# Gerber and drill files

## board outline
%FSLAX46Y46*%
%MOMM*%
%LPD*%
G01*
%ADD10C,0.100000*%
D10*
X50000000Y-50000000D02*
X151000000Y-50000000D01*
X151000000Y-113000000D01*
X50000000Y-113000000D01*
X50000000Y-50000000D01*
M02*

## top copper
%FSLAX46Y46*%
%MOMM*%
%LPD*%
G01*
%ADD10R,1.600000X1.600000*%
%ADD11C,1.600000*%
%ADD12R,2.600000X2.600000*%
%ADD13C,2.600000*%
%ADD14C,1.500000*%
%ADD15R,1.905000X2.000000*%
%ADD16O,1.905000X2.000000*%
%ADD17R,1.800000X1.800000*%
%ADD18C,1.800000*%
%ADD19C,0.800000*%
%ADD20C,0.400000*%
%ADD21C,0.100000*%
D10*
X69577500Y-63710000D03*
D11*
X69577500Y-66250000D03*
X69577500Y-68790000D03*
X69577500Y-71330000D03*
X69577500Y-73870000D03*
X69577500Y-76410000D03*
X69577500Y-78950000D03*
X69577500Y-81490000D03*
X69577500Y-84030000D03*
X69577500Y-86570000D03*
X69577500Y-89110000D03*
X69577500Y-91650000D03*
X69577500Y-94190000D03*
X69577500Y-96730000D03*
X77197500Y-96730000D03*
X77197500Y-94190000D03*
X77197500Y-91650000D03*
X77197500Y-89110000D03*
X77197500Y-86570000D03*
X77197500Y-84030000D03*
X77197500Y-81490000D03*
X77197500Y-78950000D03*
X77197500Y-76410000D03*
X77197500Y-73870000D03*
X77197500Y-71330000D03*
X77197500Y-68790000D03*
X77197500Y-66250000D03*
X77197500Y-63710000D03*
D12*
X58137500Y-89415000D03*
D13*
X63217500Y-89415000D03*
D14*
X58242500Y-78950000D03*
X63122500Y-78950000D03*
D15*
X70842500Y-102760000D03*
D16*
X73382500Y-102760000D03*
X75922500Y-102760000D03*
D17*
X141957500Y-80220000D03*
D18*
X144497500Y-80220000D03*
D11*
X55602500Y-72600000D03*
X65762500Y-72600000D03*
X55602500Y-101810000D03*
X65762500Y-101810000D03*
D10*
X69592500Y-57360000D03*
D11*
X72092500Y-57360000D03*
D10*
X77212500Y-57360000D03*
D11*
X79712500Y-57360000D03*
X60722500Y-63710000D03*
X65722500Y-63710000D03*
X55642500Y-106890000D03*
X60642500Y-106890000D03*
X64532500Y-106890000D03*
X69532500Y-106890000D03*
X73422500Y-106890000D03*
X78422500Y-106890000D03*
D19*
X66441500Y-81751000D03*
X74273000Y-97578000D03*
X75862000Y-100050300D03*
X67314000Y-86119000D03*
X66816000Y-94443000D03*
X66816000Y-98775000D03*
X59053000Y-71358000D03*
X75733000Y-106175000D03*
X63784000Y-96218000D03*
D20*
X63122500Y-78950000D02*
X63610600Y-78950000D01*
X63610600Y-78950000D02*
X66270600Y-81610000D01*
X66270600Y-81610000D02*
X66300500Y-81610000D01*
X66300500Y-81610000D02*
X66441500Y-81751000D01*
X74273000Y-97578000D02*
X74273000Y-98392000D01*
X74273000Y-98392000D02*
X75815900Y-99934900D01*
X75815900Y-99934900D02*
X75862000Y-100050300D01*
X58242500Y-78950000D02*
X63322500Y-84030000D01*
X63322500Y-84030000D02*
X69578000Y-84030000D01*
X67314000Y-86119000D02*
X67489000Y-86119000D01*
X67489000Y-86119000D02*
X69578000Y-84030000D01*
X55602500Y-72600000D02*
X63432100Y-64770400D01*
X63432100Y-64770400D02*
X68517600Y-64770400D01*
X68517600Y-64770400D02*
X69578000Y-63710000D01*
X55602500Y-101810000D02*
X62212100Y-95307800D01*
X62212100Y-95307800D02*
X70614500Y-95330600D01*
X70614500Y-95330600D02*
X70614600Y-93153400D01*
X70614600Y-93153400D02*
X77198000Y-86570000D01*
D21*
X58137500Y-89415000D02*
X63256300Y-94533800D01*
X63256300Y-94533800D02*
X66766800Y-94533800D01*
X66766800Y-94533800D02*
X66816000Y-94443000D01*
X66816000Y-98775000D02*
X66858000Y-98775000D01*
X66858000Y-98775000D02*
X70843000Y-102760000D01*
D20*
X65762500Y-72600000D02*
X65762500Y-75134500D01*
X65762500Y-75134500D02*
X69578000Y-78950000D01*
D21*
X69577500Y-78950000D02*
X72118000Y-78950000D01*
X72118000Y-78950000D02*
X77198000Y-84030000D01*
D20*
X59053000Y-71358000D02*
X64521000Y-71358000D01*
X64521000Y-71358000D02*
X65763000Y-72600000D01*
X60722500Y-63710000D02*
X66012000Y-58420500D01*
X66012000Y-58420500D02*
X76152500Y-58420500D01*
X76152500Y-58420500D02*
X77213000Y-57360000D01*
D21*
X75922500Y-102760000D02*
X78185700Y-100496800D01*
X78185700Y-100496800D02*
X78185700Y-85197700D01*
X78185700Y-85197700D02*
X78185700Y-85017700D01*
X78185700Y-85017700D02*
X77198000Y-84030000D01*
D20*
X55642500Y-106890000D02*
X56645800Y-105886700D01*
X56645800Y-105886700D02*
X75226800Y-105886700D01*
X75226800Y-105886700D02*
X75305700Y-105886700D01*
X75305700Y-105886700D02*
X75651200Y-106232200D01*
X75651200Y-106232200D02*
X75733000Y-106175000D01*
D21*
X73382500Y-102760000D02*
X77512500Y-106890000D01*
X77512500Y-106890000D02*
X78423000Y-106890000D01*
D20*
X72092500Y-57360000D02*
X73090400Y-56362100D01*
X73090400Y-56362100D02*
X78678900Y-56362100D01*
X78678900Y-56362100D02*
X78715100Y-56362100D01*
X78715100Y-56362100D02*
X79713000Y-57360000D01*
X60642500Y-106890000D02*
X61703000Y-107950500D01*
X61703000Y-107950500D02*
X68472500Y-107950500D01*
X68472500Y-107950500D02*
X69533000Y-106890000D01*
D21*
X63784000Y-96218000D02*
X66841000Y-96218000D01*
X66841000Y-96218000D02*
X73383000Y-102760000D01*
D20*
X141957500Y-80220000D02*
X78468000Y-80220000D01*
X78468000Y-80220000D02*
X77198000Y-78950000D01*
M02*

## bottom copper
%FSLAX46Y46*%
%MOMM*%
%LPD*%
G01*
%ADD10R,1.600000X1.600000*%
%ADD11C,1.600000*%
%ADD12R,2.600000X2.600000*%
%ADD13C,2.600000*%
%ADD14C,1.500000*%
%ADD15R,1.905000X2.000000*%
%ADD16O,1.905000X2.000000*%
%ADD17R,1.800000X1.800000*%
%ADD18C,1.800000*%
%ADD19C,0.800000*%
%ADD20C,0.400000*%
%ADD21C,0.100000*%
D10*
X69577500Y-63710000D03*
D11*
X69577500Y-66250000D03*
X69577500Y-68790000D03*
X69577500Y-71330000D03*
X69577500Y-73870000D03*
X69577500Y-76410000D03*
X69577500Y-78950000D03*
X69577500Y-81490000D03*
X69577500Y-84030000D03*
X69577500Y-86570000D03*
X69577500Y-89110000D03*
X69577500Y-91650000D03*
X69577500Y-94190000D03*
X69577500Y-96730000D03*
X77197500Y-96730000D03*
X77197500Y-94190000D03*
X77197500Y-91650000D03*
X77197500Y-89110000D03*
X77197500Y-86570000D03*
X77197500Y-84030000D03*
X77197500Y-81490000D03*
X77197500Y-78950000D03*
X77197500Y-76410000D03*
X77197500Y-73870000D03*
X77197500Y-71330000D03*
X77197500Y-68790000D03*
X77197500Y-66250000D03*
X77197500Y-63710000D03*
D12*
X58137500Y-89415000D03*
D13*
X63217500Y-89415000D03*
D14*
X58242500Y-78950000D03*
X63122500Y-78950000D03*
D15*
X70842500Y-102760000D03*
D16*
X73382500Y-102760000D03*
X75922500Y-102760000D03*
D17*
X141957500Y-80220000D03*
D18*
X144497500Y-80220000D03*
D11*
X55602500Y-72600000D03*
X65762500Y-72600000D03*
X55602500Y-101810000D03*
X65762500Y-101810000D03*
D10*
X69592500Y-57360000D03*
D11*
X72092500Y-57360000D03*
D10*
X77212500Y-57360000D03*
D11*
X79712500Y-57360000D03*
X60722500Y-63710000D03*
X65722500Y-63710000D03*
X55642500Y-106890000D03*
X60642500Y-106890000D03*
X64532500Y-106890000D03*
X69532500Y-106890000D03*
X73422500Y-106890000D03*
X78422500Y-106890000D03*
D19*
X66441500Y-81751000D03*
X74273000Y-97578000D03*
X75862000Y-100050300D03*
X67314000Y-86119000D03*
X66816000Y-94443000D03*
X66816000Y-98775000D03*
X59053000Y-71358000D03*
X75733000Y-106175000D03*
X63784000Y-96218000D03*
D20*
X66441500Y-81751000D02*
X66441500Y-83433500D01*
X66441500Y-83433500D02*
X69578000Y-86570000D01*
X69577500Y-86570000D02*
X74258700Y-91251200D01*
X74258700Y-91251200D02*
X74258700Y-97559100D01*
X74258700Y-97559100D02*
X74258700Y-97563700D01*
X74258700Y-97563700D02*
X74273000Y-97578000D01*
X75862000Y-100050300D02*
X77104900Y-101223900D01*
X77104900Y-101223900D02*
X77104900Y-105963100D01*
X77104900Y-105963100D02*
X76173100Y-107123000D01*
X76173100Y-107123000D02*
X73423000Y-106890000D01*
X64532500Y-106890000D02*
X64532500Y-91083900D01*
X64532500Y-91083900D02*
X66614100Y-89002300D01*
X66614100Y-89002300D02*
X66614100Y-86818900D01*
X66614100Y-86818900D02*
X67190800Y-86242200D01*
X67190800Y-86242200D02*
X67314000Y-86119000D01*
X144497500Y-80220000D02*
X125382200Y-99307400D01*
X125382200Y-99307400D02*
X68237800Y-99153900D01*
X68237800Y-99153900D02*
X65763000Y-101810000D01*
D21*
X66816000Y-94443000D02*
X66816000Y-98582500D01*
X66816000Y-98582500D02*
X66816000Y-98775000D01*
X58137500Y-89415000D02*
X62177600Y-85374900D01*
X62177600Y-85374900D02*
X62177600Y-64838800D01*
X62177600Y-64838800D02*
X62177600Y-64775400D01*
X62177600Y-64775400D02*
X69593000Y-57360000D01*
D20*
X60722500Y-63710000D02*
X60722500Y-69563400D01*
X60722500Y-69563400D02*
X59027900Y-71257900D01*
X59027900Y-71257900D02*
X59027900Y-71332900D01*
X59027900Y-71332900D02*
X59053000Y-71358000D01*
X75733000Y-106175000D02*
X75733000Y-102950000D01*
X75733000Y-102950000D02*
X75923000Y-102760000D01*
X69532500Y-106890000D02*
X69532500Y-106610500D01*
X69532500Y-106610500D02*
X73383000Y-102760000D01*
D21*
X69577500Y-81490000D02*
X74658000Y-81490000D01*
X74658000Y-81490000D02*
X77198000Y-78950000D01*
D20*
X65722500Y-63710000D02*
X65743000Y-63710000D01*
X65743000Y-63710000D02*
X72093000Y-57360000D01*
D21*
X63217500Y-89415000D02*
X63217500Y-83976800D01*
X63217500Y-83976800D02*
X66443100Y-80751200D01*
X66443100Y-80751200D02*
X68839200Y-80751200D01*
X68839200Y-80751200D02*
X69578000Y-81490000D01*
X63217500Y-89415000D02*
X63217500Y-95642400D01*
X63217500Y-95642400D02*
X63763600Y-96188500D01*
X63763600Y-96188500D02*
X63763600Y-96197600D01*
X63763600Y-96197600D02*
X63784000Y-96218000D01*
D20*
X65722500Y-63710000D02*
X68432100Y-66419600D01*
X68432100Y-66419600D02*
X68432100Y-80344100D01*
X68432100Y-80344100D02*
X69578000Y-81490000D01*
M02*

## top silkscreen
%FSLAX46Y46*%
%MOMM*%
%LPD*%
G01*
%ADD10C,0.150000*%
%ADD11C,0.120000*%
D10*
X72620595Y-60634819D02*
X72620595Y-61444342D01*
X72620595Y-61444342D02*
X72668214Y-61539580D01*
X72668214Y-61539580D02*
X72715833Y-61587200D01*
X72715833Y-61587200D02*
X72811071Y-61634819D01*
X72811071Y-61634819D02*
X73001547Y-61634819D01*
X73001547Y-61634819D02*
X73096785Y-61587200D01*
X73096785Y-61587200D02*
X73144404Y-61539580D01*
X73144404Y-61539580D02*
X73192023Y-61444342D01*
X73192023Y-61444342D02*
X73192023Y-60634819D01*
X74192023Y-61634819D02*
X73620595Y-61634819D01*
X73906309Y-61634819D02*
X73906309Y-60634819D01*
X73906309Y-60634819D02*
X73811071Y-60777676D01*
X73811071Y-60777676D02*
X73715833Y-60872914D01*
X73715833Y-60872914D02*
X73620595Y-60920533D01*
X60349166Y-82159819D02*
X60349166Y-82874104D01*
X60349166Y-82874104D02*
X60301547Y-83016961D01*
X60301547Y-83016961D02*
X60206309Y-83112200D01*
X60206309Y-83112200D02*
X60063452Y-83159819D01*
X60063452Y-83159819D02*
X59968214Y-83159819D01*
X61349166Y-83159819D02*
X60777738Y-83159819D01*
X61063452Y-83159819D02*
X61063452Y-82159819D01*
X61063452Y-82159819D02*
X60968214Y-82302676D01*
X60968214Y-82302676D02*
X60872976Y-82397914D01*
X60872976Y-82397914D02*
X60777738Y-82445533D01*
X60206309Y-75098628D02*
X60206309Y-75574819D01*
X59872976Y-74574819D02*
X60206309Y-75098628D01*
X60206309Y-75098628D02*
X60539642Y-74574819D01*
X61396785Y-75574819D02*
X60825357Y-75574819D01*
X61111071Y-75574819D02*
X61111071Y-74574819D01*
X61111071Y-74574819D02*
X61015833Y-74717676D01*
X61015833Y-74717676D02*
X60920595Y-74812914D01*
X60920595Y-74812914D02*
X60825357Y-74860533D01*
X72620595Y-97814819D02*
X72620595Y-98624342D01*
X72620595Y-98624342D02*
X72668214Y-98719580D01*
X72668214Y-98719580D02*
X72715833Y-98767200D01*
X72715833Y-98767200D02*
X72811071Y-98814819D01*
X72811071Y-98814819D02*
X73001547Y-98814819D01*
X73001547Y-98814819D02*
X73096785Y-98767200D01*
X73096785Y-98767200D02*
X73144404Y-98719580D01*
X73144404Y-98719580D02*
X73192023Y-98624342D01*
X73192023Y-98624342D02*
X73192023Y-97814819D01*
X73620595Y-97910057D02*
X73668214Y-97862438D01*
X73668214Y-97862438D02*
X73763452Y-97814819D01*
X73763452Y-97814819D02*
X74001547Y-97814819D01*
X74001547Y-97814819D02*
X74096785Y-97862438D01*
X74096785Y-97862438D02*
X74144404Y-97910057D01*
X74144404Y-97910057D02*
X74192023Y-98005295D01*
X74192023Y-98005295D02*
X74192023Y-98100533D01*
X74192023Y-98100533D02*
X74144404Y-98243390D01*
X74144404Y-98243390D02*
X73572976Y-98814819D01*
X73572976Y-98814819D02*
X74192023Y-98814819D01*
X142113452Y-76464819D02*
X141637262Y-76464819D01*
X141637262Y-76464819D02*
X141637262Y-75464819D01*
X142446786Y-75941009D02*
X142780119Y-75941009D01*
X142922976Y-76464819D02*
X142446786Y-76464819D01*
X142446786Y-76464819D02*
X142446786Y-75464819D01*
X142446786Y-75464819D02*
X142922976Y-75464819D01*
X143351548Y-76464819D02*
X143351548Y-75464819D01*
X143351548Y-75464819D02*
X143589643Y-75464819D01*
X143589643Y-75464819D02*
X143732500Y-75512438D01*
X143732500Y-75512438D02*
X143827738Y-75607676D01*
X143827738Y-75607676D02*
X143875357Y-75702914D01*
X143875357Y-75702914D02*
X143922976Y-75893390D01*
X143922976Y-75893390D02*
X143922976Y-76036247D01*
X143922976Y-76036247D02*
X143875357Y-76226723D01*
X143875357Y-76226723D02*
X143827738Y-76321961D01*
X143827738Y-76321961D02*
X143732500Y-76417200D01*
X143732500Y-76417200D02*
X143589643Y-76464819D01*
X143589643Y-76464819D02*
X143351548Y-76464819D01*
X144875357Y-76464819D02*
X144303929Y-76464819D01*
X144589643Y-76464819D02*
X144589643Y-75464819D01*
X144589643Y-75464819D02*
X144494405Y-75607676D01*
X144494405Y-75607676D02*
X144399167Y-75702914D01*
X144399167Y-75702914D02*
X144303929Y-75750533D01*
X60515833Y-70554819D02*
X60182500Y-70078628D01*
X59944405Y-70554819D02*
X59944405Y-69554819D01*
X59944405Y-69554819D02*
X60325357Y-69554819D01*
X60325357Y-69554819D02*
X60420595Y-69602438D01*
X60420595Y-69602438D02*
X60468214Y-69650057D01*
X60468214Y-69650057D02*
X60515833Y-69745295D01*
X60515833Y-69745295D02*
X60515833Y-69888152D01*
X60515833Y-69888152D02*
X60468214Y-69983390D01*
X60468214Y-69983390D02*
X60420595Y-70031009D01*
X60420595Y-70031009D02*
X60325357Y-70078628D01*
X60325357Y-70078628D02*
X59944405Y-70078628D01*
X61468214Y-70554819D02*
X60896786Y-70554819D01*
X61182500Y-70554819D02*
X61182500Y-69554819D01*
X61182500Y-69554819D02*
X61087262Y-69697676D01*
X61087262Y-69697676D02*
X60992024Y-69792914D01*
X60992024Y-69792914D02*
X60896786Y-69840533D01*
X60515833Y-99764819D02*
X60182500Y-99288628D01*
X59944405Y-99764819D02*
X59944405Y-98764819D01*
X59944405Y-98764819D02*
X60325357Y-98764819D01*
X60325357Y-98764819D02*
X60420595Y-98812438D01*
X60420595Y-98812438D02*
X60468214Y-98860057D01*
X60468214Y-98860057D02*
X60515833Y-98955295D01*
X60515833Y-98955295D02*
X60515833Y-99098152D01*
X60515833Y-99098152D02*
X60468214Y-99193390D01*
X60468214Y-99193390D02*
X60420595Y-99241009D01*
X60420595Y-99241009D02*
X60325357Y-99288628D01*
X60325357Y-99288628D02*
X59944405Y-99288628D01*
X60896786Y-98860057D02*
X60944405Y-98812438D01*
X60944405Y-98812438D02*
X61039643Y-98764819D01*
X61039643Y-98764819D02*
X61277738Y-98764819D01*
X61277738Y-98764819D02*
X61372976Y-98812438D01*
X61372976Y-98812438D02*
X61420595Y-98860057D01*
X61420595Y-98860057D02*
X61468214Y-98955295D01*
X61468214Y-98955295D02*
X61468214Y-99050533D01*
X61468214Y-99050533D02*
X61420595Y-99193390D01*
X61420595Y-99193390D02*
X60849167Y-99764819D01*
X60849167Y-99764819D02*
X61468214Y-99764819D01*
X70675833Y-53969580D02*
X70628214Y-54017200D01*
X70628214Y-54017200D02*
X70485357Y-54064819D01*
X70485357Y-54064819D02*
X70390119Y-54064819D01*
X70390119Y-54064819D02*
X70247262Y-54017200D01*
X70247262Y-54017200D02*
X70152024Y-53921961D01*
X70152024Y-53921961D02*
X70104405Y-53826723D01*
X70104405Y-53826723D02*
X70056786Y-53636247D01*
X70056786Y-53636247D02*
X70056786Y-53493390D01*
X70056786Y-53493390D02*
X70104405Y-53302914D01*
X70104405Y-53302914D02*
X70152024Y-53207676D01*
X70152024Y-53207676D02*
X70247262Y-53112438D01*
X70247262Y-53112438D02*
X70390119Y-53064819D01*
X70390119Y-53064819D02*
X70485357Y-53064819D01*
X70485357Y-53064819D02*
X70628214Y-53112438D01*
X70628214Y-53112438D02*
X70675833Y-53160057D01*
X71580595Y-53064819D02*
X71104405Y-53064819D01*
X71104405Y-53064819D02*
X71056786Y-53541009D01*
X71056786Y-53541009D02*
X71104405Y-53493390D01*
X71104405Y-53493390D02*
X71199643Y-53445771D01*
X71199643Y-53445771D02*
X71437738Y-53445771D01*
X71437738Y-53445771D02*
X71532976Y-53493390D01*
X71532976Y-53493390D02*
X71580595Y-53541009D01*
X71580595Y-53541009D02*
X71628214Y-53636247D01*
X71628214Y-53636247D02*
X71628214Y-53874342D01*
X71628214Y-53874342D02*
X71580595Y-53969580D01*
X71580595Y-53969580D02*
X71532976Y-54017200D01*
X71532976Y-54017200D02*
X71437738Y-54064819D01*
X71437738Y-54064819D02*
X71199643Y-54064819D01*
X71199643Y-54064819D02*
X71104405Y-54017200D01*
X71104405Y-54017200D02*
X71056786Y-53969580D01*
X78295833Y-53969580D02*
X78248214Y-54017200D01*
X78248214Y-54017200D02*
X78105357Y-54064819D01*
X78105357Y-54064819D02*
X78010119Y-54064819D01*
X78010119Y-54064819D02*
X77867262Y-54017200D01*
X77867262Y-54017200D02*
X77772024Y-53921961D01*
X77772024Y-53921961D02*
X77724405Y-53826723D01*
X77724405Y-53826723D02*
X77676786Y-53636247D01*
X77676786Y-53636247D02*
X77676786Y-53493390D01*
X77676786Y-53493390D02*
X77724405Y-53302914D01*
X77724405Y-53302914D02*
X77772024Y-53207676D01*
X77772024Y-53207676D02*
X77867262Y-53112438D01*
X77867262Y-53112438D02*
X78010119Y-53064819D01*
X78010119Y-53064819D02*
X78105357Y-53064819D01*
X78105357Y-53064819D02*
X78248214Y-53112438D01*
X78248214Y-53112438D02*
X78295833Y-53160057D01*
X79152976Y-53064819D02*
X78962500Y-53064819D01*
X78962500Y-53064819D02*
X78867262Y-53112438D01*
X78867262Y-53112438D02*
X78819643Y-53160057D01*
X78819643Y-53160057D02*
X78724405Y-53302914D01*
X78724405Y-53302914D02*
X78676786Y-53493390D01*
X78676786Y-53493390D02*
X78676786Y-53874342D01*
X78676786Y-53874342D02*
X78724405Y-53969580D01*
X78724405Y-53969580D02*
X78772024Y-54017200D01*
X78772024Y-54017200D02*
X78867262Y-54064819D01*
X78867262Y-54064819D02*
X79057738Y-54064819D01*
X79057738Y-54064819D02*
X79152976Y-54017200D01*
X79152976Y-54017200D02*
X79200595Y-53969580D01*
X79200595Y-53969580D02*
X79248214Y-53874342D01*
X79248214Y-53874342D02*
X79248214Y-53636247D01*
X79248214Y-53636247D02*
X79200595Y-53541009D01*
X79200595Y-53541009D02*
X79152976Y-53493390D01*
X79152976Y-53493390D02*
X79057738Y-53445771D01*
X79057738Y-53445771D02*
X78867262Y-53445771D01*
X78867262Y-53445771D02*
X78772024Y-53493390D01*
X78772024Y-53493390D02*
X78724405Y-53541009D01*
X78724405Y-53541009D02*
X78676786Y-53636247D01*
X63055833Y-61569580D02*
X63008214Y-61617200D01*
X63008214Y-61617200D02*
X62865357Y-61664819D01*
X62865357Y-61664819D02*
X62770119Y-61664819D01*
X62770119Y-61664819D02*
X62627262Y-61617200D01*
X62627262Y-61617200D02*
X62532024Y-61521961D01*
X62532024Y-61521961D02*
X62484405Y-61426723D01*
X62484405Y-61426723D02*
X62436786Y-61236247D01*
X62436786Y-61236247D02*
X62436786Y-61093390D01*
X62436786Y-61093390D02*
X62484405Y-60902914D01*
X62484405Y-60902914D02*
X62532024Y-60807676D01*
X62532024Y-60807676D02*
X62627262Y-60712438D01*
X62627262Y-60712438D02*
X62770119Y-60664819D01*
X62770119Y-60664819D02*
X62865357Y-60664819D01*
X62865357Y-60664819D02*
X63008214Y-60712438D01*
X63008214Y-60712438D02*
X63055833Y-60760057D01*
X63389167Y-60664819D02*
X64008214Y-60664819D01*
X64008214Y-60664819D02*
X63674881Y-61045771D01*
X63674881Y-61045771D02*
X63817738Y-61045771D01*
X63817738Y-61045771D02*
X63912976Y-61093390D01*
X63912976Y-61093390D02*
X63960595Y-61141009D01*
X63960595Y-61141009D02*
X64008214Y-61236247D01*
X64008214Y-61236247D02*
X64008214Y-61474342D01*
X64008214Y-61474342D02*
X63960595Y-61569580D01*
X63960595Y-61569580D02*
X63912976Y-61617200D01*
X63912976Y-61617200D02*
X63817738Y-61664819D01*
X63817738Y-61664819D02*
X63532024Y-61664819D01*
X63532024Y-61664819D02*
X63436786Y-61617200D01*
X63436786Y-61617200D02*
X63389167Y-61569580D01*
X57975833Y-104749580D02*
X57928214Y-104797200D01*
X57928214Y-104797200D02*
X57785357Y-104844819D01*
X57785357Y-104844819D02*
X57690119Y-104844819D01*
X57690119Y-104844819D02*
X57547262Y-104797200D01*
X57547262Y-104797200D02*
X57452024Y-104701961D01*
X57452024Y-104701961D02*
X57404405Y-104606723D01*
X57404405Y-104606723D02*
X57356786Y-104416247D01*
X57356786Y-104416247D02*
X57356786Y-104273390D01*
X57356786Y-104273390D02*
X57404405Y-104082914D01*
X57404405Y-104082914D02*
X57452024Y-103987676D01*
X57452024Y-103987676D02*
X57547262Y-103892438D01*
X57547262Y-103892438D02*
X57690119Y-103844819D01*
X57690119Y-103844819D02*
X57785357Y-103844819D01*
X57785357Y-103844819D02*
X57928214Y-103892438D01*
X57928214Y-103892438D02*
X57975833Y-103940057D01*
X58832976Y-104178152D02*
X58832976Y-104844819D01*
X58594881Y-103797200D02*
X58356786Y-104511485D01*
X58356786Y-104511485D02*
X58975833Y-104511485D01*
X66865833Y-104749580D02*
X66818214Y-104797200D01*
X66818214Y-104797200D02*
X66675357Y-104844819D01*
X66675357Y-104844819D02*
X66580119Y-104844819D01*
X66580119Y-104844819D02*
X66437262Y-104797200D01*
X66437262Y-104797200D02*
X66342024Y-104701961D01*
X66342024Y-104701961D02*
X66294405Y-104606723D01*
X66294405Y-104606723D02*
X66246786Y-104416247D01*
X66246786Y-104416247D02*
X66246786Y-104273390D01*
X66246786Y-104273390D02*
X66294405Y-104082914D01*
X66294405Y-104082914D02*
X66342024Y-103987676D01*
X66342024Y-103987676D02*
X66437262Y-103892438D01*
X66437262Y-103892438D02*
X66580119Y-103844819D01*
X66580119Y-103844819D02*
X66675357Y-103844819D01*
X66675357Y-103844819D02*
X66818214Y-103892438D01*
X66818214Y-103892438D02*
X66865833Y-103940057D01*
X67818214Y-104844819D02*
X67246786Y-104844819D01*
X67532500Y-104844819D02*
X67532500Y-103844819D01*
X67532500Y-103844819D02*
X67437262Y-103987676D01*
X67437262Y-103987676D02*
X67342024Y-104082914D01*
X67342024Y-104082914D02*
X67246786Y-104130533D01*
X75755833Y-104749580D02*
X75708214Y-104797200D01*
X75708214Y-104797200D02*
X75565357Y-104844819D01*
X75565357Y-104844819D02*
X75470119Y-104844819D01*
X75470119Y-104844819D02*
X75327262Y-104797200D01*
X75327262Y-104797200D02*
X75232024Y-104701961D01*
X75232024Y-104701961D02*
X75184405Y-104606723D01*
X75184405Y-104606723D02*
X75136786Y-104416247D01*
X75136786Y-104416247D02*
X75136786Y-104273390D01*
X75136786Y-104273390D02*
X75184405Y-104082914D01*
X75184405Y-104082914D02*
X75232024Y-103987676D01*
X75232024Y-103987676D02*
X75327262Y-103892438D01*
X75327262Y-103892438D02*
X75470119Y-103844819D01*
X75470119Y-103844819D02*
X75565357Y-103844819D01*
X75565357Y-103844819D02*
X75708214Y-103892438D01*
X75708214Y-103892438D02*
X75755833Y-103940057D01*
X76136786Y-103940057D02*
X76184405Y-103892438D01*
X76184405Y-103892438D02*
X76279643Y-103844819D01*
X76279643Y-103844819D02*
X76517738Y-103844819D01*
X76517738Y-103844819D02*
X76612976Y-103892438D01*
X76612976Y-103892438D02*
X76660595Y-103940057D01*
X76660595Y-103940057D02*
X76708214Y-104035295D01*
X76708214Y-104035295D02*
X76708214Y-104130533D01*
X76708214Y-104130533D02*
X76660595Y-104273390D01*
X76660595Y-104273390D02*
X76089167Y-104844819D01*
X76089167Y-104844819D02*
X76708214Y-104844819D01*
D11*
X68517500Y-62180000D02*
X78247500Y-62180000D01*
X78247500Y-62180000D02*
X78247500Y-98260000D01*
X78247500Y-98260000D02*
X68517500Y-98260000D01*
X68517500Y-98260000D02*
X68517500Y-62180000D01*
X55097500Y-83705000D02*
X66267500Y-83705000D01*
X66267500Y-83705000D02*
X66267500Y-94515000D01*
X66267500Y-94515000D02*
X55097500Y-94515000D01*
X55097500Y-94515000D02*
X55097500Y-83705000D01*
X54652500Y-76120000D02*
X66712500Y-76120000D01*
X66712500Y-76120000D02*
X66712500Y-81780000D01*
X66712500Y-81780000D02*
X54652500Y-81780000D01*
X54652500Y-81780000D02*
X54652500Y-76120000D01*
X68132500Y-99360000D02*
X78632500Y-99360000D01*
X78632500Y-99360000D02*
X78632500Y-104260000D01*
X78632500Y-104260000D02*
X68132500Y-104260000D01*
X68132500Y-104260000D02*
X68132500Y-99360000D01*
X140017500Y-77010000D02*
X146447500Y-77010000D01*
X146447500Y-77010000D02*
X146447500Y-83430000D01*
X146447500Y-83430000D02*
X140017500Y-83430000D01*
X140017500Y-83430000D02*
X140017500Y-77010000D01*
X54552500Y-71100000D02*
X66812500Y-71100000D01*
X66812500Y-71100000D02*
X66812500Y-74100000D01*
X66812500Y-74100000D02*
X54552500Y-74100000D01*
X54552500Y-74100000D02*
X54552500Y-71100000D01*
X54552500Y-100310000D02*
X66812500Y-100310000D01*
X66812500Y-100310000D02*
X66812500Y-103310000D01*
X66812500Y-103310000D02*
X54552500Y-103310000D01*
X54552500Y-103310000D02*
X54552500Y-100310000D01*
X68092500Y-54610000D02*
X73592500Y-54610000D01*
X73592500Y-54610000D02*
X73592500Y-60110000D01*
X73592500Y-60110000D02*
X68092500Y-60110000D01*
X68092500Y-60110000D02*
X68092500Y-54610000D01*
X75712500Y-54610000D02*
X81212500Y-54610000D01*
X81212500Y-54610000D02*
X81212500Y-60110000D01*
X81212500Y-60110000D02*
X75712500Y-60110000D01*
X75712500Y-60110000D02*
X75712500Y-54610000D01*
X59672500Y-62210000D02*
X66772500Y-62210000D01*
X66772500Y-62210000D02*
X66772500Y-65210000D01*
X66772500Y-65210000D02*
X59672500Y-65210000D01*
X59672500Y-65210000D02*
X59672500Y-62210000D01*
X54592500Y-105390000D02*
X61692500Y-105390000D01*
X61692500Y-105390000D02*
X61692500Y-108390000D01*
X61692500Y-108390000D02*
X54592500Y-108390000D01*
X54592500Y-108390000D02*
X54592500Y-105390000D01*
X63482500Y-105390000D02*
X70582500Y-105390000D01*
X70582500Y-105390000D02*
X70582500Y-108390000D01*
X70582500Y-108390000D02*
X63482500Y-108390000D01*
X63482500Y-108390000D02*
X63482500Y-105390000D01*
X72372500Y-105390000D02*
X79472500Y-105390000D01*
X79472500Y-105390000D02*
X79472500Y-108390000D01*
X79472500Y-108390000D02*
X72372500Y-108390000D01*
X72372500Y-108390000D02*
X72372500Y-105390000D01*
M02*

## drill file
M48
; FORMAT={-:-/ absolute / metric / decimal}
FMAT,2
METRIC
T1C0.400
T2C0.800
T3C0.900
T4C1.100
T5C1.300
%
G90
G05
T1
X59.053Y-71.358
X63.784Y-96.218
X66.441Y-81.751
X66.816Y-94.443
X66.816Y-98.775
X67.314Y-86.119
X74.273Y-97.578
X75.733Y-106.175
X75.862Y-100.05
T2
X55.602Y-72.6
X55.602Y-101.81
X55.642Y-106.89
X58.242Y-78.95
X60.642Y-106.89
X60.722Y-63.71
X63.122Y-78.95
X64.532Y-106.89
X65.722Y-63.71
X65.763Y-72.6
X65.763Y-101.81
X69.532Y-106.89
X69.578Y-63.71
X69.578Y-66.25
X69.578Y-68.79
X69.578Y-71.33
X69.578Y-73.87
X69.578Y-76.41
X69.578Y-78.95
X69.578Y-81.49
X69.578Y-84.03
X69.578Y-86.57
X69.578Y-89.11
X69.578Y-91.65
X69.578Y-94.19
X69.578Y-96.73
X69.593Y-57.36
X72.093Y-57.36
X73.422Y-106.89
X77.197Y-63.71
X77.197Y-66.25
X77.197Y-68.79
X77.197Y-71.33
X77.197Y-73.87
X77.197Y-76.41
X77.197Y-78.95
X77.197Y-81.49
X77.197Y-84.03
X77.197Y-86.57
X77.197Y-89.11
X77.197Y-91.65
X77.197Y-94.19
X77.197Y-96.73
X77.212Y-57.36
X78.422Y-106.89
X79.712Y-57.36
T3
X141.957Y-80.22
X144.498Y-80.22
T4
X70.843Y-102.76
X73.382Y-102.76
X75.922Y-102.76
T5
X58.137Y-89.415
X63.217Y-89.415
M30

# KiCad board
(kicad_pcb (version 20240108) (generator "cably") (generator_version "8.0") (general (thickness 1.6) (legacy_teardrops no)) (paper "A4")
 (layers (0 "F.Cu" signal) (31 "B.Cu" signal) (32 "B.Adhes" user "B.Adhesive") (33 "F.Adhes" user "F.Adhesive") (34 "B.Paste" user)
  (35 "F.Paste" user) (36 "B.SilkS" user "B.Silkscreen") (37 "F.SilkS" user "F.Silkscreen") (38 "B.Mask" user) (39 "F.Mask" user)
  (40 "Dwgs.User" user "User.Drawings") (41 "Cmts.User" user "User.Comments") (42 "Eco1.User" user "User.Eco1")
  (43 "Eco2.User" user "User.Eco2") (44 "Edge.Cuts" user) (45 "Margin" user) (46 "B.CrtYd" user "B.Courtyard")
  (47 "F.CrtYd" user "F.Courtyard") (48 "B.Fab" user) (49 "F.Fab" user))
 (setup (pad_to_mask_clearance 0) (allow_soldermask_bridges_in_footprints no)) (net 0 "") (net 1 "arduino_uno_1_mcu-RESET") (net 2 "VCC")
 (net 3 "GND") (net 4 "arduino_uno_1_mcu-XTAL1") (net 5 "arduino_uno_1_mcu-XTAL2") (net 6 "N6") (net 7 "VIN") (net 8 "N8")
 (gr_rect (start 50 50) (end 151 113) (stroke (width 0.1) (type default)) (fill none) (layer "Edge.Cuts"))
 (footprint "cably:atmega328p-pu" (layer "F.Cu") (at 73.3825 80.22)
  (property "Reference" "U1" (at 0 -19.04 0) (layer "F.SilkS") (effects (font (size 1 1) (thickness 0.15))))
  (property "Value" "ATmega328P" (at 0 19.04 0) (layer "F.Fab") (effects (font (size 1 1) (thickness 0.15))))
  (fp_line (start -4.865 -18.04) (end 4.865 -18.04) (stroke (width 0.12) (type solid)) (layer "F.SilkS"))
  (fp_line (start 4.865 -18.04) (end 4.865 18.04) (stroke (width 0.12) (type solid)) (layer "F.SilkS"))
  (fp_line (start 4.865 18.04) (end -4.865 18.04) (stroke (width 0.12) (type solid)) (layer "F.SilkS"))
  (fp_line (start -4.865 18.04) (end -4.865 -18.04) (stroke (width 0.12) (type solid)) (layer "F.SilkS"))
  (pad "1" thru_hole rect (at -3.805 -16.51) (size 1.6 1.6) (drill 0.8) (layers "*.Cu" "*.Mask") (remove_unused_layers no)
   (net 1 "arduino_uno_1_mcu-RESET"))
  (pad "2" thru_hole circle (at -3.805 -13.97) (size 1.6 1.6) (drill 0.8) (layers "*.Cu" "*.Mask") (remove_unused_layers no))
  (pad "3" thru_hole circle (at -3.805 -11.43) (size 1.6 1.6) (drill 0.8) (layers "*.Cu" "*.Mask") (remove_unused_layers no))
  (pad "4" thru_hole circle (at -3.805 -8.89) (size 1.6 1.6) (drill 0.8) (layers "*.Cu" "*.Mask") (remove_unused_layers no))
  (pad "5" thru_hole circle (at -3.805 -6.35) (size 1.6 1.6) (drill 0.8) (layers "*.Cu" "*.Mask") (remove_unused_layers no))
  (pad "6" thru_hole circle (at -3.805 -3.81) (size 1.6 1.6) (drill 0.8) (layers "*.Cu" "*.Mask") (remove_unused_layers no))
  (pad "7" thru_hole circle (at -3.805 -1.27) (size 1.6 1.6) (drill 0.8) (layers "*.Cu" "*.Mask") (remove_unused_layers no) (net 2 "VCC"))
  (pad "8" thru_hole circle (at -3.805 1.27) (size 1.6 1.6) (drill 0.8) (layers "*.Cu" "*.Mask") (remove_unused_layers no) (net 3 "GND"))
  (pad "9" thru_hole circle (at -3.805 3.81) (size 1.6 1.6) (drill 0.8) (layers "*.Cu" "*.Mask") (remove_unused_layers no)
   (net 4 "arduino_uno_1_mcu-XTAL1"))
  (pad "10" thru_hole circle (at -3.805 6.35) (size 1.6 1.6) (drill 0.8) (layers "*.Cu" "*.Mask") (remove_unused_layers no)
   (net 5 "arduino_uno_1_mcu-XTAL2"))
  (pad "11" thru_hole circle (at -3.805 8.89) (size 1.6 1.6) (drill 0.8) (layers "*.Cu" "*.Mask") (remove_unused_layers no))
  (pad "12" thru_hole circle (at -3.805 11.43) (size 1.6 1.6) (drill 0.8) (layers "*.Cu" "*.Mask") (remove_unused_layers no))
  (pad "13" thru_hole circle (at -3.805 13.97) (size 1.6 1.6) (drill 0.8) (layers "*.Cu" "*.Mask") (remove_unused_layers no))
  (pad "14" thru_hole circle (at -3.805 16.51) (size 1.6 1.6) (drill 0.8) (layers "*.Cu" "*.Mask") (remove_unused_layers no))
  (pad "15" thru_hole circle (at 3.815 16.51) (size 1.6 1.6) (drill 0.8) (layers "*.Cu" "*.Mask") (remove_unused_layers no))
  (pad "16" thru_hole circle (at 3.815 13.97) (size 1.6 1.6) (drill 0.8) (layers "*.Cu" "*.Mask") (remove_unused_layers no))
  (pad "17" thru_hole circle (at 3.815 11.43) (size 1.6 1.6) (drill 0.8) (layers "*.Cu" "*.Mask") (remove_unused_layers no))
  (pad "18" thru_hole circle (at 3.815 8.89) (size 1.6 1.6) (drill 0.8) (layers "*.Cu" "*.Mask") (remove_unused_layers no))
  (pad "19" thru_hole circle (at 3.815 6.35) (size 1.6 1.6) (drill 0.8) (layers "*.Cu" "*.Mask") (remove_unused_layers no) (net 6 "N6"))
  (pad "20" thru_hole circle (at 3.815 3.81) (size 1.6 1.6) (drill 0.8) (layers "*.Cu" "*.Mask") (remove_unused_layers no) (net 2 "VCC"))
  (pad "21" thru_hole circle (at 3.815 1.27) (size 1.6 1.6) (drill 0.8) (layers "*.Cu" "*.Mask") (remove_unused_layers no))
  (pad "22" thru_hole circle (at 3.815 -1.27) (size 1.6 1.6) (drill 0.8) (layers "*.Cu" "*.Mask") (remove_unused_layers no) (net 3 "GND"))
  (pad "23" thru_hole circle (at 3.815 -3.81) (size 1.6 1.6) (drill 0.8) (layers "*.Cu" "*.Mask") (remove_unused_layers no))
  (pad "24" thru_hole circle (at 3.815 -6.35) (size 1.6 1.6) (drill 0.8) (layers "*.Cu" "*.Mask") (remove_unused_layers no))
  (pad "25" thru_hole circle (at 3.815 -8.89) (size 1.6 1.6) (drill 0.8) (layers "*.Cu" "*.Mask") (remove_unused_layers no))
  (pad "26" thru_hole circle (at 3.815 -11.43) (size 1.6 1.6) (drill 0.8) (layers "*.Cu" "*.Mask") (remove_unused_layers no))
  (pad "27" thru_hole circle (at 3.815 -13.97) (size 1.6 1.6) (drill 0.8) (layers "*.Cu" "*.Mask") (remove_unused_layers no))
  (pad "28" thru_hole circle (at 3.815 -16.51) (size 1.6 1.6) (drill 0.8) (layers "*.Cu" "*.Mask") (remove_unused_layers no)))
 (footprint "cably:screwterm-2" (layer "F.Cu") (at 60.6825 89.11)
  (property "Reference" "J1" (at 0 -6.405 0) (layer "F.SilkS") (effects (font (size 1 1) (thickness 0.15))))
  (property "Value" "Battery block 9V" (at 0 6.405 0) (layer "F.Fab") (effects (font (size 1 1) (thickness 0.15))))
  (fp_line (start -5.585 -5.405) (end 5.585 -5.405) (stroke (width 0.12) (type solid)) (layer "F.SilkS"))
  (fp_line (start 5.585 -5.405) (end 5.585 5.405) (stroke (width 0.12) (type solid)) (layer "F.SilkS"))
  (fp_line (start 5.585 5.405) (end -5.585 5.405) (stroke (width 0.12) (type solid)) (layer "F.SilkS"))
  (fp_line (start -5.585 5.405) (end -5.585 -5.405) (stroke (width 0.12) (type solid)) (layer "F.SilkS"))
  (pad "1" thru_hole rect (at -2.545 0.305) (size 2.6 2.6) (drill 1.3) (layers "*.Cu" "*.Mask") (remove_unused_layers no) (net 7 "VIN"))
  (pad "2" thru_hole circle (at 2.535 0.305) (size 2.6 2.6) (drill 1.3) (layers "*.Cu" "*.Mask") (remove_unused_layers no) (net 3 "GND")))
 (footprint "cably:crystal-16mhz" (layer "F.Cu") (at 60.6825 78.95)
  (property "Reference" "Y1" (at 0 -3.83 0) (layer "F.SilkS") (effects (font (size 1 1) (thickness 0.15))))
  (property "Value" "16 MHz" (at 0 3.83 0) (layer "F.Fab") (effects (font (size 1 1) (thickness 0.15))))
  (fp_line (start -6.03 -2.83) (end 6.03 -2.83) (stroke (width 0.12) (type solid)) (layer "F.SilkS"))
  (fp_line (start 6.03 -2.83) (end 6.03 2.83) (stroke (width 0.12) (type solid)) (layer "F.SilkS"))
  (fp_line (start 6.03 2.83) (end -6.03 2.83) (stroke (width 0.12) (type solid)) (layer "F.SilkS"))
  (fp_line (start -6.03 2.83) (end -6.03 -2.83) (stroke (width 0.12) (type solid)) (layer "F.SilkS"))
  (pad "1" thru_hole circle (at -2.44 0) (size 1.5 1.5) (drill 0.8) (layers "*.Cu" "*.Mask") (remove_unused_layers no)
   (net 4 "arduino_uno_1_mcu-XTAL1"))
  (pad "2" thru_hole circle (at 2.44 0) (size 1.5 1.5) (drill 0.8) (layers "*.Cu" "*.Mask") (remove_unused_layers no)
   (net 5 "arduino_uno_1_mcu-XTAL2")))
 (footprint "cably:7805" (layer "F.Cu") (at 73.3825 101.81)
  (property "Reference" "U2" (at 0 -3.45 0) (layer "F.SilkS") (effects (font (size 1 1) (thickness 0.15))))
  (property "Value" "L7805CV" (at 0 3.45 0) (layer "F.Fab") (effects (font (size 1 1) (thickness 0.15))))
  (fp_line (start -5.25 -2.45) (end 5.25 -2.45) (stroke (width 0.12) (type solid)) (layer "F.SilkS"))
  (fp_line (start 5.25 -2.45) (end 5.25 2.45) (stroke (width 0.12) (type solid)) (layer "F.SilkS"))
  (fp_line (start 5.25 2.45) (end -5.25 2.45) (stroke (width 0.12) (type solid)) (layer "F.SilkS"))
  (fp_line (start -5.25 2.45) (end -5.25 -2.45) (stroke (width 0.12) (type solid)) (layer "F.SilkS"))
  (pad "1" thru_hole rect (at -2.54 0.95) (size 1.905 2) (drill 1.1) (layers "*.Cu" "*.Mask") (remove_unused_layers no) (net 7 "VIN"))
  (pad "2" thru_hole oval (at 0 0.95) (size 1.905 2) (drill 1.1) (layers "*.Cu" "*.Mask") (remove_unused_layers no) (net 3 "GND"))
  (pad "3" thru_hole oval (at 2.54 0.95) (size 1.905 2) (drill 1.1) (layers "*.Cu" "*.Mask") (remove_unused_layers no) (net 2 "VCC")))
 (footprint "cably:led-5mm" (layer "F.Cu") (at 143.2325 80.22)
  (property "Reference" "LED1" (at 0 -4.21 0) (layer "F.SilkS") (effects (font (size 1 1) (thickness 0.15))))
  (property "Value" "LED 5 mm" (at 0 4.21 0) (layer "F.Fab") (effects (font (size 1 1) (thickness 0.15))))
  (fp_line (start -3.215 -3.21) (end 3.215 -3.21) (stroke (width 0.12) (type solid)) (layer "F.SilkS"))
  (fp_line (start 3.215 -3.21) (end 3.215 3.21) (stroke (width 0.12) (type solid)) (layer "F.SilkS"))
  (fp_line (start 3.215 3.21) (end -3.215 3.21) (stroke (width 0.12) (type solid)) (layer "F.SilkS"))
  (fp_line (start -3.215 3.21) (end -3.215 -3.21) (stroke (width 0.12) (type solid)) (layer "F.SilkS"))
  (pad "1" thru_hole rect (at -1.275 0) (size 1.8 1.8) (drill 0.9) (layers "*.Cu" "*.Mask") (remove_unused_layers no) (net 3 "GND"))
  (pad "2" thru_hole circle (at 1.265 0) (size 1.8 1.8) (drill 0.9) (layers "*.Cu" "*.Mask") (remove_unused_layers no) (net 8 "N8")))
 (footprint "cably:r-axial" (layer "F.Cu") (at 60.6825 72.6)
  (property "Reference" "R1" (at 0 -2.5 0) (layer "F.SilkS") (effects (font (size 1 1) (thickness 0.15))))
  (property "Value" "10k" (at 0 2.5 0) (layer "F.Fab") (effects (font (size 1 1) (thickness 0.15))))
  (fp_line (start -6.13 -1.5) (end 6.13 -1.5) (stroke (width 0.12) (type solid)) (layer "F.SilkS"))
  (fp_line (start 6.13 -1.5) (end 6.13 1.5) (stroke (width 0.12) (type solid)) (layer "F.SilkS"))
  (fp_line (start 6.13 1.5) (end -6.13 1.5) (stroke (width 0.12) (type solid)) (layer "F.SilkS"))
  (fp_line (start -6.13 1.5) (end -6.13 -1.5) (stroke (width 0.12) (type solid)) (layer "F.SilkS"))
  (pad "1" thru_hole circle (at -5.08 0) (size 1.6 1.6) (drill 0.8) (layers "*.Cu" "*.Mask") (remove_unused_layers no)
   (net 1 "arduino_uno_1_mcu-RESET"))
  (pad "2" thru_hole circle (at 5.08 0) (size 1.6 1.6) (drill 0.8) (layers "*.Cu" "*.Mask") (remove_unused_layers no) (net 2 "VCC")))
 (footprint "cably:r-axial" (layer "F.Cu") (at 60.6825 101.81)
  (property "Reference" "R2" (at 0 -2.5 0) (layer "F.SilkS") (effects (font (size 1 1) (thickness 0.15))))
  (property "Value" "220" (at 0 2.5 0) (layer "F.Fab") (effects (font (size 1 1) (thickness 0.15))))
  (fp_line (start -6.13 -1.5) (end 6.13 -1.5) (stroke (width 0.12) (type solid)) (layer "F.SilkS"))
  (fp_line (start 6.13 -1.5) (end 6.13 1.5) (stroke (width 0.12) (type solid)) (layer "F.SilkS"))
  (fp_line (start 6.13 1.5) (end -6.13 1.5) (stroke (width 0.12) (type solid)) (layer "F.SilkS"))
  (fp_line (start -6.13 1.5) (end -6.13 -1.5) (stroke (width 0.12) (type solid)) (layer "F.SilkS"))
  (pad "1" thru_hole circle (at -5.08 0) (size 1.6 1.6) (drill 0.8) (layers "*.Cu" "*.Mask") (remove_unused_layers no) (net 6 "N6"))
  (pad "2" thru_hole circle (at 5.08 0) (size 1.6 1.6) (drill 0.8) (layers "*.Cu" "*.Mask") (remove_unused_layers no) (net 8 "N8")))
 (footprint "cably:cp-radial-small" (layer "F.Cu") (at 70.8425 57.36)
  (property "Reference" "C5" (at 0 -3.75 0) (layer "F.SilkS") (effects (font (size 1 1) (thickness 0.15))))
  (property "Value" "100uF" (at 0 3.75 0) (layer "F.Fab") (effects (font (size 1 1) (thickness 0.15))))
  (fp_line (start -2.75 -2.75) (end 2.75 -2.75) (stroke (width 0.12) (type solid)) (layer "F.SilkS"))
  (fp_line (start 2.75 -2.75) (end 2.75 2.75) (stroke (width 0.12) (type solid)) (layer "F.SilkS"))
  (fp_line (start 2.75 2.75) (end -2.75 2.75) (stroke (width 0.12) (type solid)) (layer "F.SilkS"))
  (fp_line (start -2.75 2.75) (end -2.75 -2.75) (stroke (width 0.12) (type solid)) (layer "F.SilkS"))
  (pad "1" thru_hole rect (at -1.25 0) (size 1.6 1.6) (drill 0.8) (layers "*.Cu" "*.Mask") (remove_unused_layers no) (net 7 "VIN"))
  (pad "2" thru_hole circle (at 1.25 0) (size 1.6 1.6) (drill 0.8) (layers "*.Cu" "*.Mask") (remove_unused_layers no) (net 3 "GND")))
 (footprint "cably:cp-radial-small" (layer "F.Cu") (at 78.4625 57.36)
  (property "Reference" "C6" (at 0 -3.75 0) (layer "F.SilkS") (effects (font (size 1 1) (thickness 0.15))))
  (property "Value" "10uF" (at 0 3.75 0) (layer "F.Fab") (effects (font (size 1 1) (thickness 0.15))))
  (fp_line (start -2.75 -2.75) (end 2.75 -2.75) (stroke (width 0.12) (type solid)) (layer "F.SilkS"))
  (fp_line (start 2.75 -2.75) (end 2.75 2.75) (stroke (width 0.12) (type solid)) (layer "F.SilkS"))
  (fp_line (start 2.75 2.75) (end -2.75 2.75) (stroke (width 0.12) (type solid)) (layer "F.SilkS"))
  (fp_line (start -2.75 2.75) (end -2.75 -2.75) (stroke (width 0.12) (type solid)) (layer "F.SilkS"))
  (pad "1" thru_hole rect (at -1.25 0) (size 1.6 1.6) (drill 0.8) (layers "*.Cu" "*.Mask") (remove_unused_layers no) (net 2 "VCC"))
  (pad "2" thru_hole circle (at 1.25 0) (size 1.6 1.6) (drill 0.8) (layers "*.Cu" "*.Mask") (remove_unused_layers no) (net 3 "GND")))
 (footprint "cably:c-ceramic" (layer "F.Cu") (at 63.2225 63.71)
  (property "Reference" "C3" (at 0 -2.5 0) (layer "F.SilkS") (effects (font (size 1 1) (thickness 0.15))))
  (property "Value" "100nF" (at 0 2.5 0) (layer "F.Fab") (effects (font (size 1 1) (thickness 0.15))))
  (fp_line (start -3.55 -1.5) (end 3.55 -1.5) (stroke (width 0.12) (type solid)) (layer "F.SilkS"))
  (fp_line (start 3.55 -1.5) (end 3.55 1.5) (stroke (width 0.12) (type solid)) (layer "F.SilkS"))
  (fp_line (start 3.55 1.5) (end -3.55 1.5) (stroke (width 0.12) (type solid)) (layer "F.SilkS"))
  (fp_line (start -3.55 1.5) (end -3.55 -1.5) (stroke (width 0.12) (type solid)) (layer "F.SilkS"))
  (pad "1" thru_hole circle (at -2.5 0) (size 1.6 1.6) (drill 0.8) (layers "*.Cu" "*.Mask") (remove_unused_layers no) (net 2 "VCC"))
  (pad "2" thru_hole circle (at 2.5 0) (size 1.6 1.6) (drill 0.8) (layers "*.Cu" "*.Mask") (remove_unused_layers no) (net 3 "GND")))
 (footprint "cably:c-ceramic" (layer "F.Cu") (at 58.1425 106.89)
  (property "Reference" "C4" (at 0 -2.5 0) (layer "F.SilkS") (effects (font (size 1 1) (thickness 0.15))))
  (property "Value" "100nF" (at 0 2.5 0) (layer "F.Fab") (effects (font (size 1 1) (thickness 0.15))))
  (fp_line (start -3.55 -1.5) (end 3.55 -1.5) (stroke (width 0.12) (type solid)) (layer "F.SilkS"))
  (fp_line (start 3.55 -1.5) (end 3.55 1.5) (stroke (width 0.12) (type solid)) (layer "F.SilkS"))
  (fp_line (start 3.55 1.5) (end -3.55 1.5) (stroke (width 0.12) (type solid)) (layer "F.SilkS"))
  (fp_line (start -3.55 1.5) (end -3.55 -1.5) (stroke (width 0.12) (type solid)) (layer "F.SilkS"))
  (pad "1" thru_hole circle (at -2.5 0) (size 1.6 1.6) (drill 0.8) (layers "*.Cu" "*.Mask") (remove_unused_layers no) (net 2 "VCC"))
  (pad "2" thru_hole circle (at 2.5 0) (size 1.6 1.6) (drill 0.8) (layers "*.Cu" "*.Mask") (remove_unused_layers no) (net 3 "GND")))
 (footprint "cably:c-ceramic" (layer "F.Cu") (at 67.0325 106.89)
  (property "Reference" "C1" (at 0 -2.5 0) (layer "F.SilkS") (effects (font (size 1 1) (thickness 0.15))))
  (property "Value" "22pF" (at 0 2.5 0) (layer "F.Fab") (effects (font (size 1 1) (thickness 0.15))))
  (fp_line (start -3.55 -1.5) (end 3.55 -1.5) (stroke (width 0.12) (type solid)) (layer "F.SilkS"))
  (fp_line (start 3.55 -1.5) (end 3.55 1.5) (stroke (width 0.12) (type solid)) (layer "F.SilkS"))
  (fp_line (start 3.55 1.5) (end -3.55 1.5) (stroke (width 0.12) (type solid)) (layer "F.SilkS"))
  (fp_line (start -3.55 1.5) (end -3.55 -1.5) (stroke (width 0.12) (type solid)) (layer "F.SilkS"))
  (pad "1" thru_hole circle (at -2.5 0) (size 1.6 1.6) (drill 0.8) (layers "*.Cu" "*.Mask") (remove_unused_layers no)
   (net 4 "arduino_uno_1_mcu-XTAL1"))
  (pad "2" thru_hole circle (at 2.5 0) (size 1.6 1.6) (drill 0.8) (layers "*.Cu" "*.Mask") (remove_unused_layers no) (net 3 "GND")))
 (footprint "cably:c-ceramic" (layer "F.Cu") (at 75.9225 106.89)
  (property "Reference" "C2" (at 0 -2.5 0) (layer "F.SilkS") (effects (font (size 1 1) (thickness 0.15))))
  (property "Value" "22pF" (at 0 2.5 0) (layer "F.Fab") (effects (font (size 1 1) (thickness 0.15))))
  (fp_line (start -3.55 -1.5) (end 3.55 -1.5) (stroke (width 0.12) (type solid)) (layer "F.SilkS"))
  (fp_line (start 3.55 -1.5) (end 3.55 1.5) (stroke (width 0.12) (type solid)) (layer "F.SilkS"))
  (fp_line (start 3.55 1.5) (end -3.55 1.5) (stroke (width 0.12) (type solid)) (layer "F.SilkS"))
  (fp_line (start -3.55 1.5) (end -3.55 -1.5) (stroke (width 0.12) (type solid)) (layer "F.SilkS"))
  (pad "1" thru_hole circle (at -2.5 0) (size 1.6 1.6) (drill 0.8) (layers "*.Cu" "*.Mask") (remove_unused_layers no)
   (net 5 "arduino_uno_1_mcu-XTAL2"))
  (pad "2" thru_hole circle (at 2.5 0) (size 1.6 1.6) (drill 0.8) (layers "*.Cu" "*.Mask") (remove_unused_layers no) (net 3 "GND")))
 (segment (start 63.1225 78.95) (end 63.6106 78.95) (width 0.4) (layer "F.Cu") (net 5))
 (segment (start 63.6106 78.95) (end 66.2706 81.61) (width 0.4) (layer "F.Cu") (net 5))
 (segment (start 66.2706 81.61) (end 66.3005 81.61) (width 0.4) (layer "F.Cu") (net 5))
 (segment (start 66.3005 81.61) (end 66.4415 81.751) (width 0.4) (layer "F.Cu") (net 5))
 (segment (start 66.4415 81.751) (end 66.4415 83.4335) (width 0.4) (layer "B.Cu") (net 5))
 (segment (start 66.4415 83.4335) (end 69.578 86.57) (width 0.4) (layer "B.Cu") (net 5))
 (segment (start 69.5775 86.57) (end 74.2587 91.2512) (width 0.4) (layer "B.Cu") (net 5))
 (segment (start 74.2587 91.2512) (end 74.2587 97.5591) (width 0.4) (layer "B.Cu") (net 5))
 (segment (start 74.2587 97.5591) (end 74.2587 97.5637) (width 0.4) (layer "B.Cu") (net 5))
 (segment (start 74.2587 97.5637) (end 74.273 97.578) (width 0.4) (layer "B.Cu") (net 5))
 (segment (start 74.273 97.578) (end 74.273 98.392) (width 0.4) (layer "F.Cu") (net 5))
 (segment (start 74.273 98.392) (end 75.8159 99.9349) (width 0.4) (layer "F.Cu") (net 5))
 (segment (start 75.8159 99.9349) (end 75.862 100.0503) (width 0.4) (layer "F.Cu") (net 5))
 (segment (start 75.862 100.0503) (end 77.1049 101.2239) (width 0.4) (layer "B.Cu") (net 5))
 (segment (start 77.1049 101.2239) (end 77.1049 105.9631) (width 0.4) (layer "B.Cu") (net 5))
 (segment (start 77.1049 105.9631) (end 76.1731 107.123) (width 0.4) (layer "B.Cu") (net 5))
 (segment (start 76.1731 107.123) (end 73.423 106.89) (width 0.4) (layer "B.Cu") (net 5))
 (segment (start 58.2425 78.95) (end 63.3225 84.03) (width 0.4) (layer "F.Cu") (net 4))
 (segment (start 63.3225 84.03) (end 69.578 84.03) (width 0.4) (layer "F.Cu") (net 4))
 (segment (start 64.5325 106.89) (end 64.5325 91.0839) (width 0.4) (layer "B.Cu") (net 4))
 (segment (start 64.5325 91.0839) (end 66.6141 89.0023) (width 0.4) (layer "B.Cu") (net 4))
 (segment (start 66.6141 89.0023) (end 66.6141 86.8189) (width 0.4) (layer "B.Cu") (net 4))
 (segment (start 66.6141 86.8189) (end 67.1908 86.2422) (width 0.4) (layer "B.Cu") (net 4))
 (segment (start 67.1908 86.2422) (end 67.314 86.119) (width 0.4) (layer "B.Cu") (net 4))
 (segment (start 67.314 86.119) (end 67.489 86.119) (width 0.4) (layer "F.Cu") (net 4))
 (segment (start 67.489 86.119) (end 69.578 84.03) (width 0.4) (layer "F.Cu") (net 4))
 (segment (start 55.6025 72.6) (end 63.4321 64.7704) (width 0.4) (layer "F.Cu") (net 1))
 (segment (start 63.4321 64.7704) (end 68.5176 64.7704) (width 0.4) (layer "F.Cu") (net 1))
 (segment (start 68.5176 64.7704) (end 69.578 63.71) (width 0.4) (layer "F.Cu") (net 1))
 (segment (start 55.6025 101.81) (end 62.2121 95.3078) (width 0.4) (layer "F.Cu") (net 6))
 (segment (start 62.2121 95.3078) (end 70.6145 95.3306) (width 0.4) (layer "F.Cu") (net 6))
 (segment (start 70.6145 95.3306) (end 70.6146 93.1534) (width 0.4) (layer "F.Cu") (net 6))
 (segment (start 70.6146 93.1534) (end 77.198 86.57) (width 0.4) (layer "F.Cu") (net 6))
 (segment (start 144.4975 80.22) (end 125.3822 99.3074) (width 0.4) (layer "B.Cu") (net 8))
 (segment (start 125.3822 99.3074) (end 68.2378 99.1539) (width 0.4) (layer "B.Cu") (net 8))
 (segment (start 68.2378 99.1539) (end 65.763 101.81) (width 0.4) (layer "B.Cu") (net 8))
 (segment (start 58.1375 89.415) (end 63.2563 94.5338) (width 0.1) (layer "F.Cu") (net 7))
 (segment (start 63.2563 94.5338) (end 66.7668 94.5338) (width 0.1) (layer "F.Cu") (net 7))
 (segment (start 66.7668 94.5338) (end 66.816 94.443) (width 0.1) (layer "F.Cu") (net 7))
 (segment (start 66.816 94.443) (end 66.816 98.5825) (width 0.1) (layer "B.Cu") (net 7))
 (segment (start 66.816 98.5825) (end 66.816 98.775) (width 0.1) (layer "B.Cu") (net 7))
 (segment (start 66.816 98.775) (end 66.858 98.775) (width 0.1) (layer "F.Cu") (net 7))
 (segment (start 66.858 98.775) (end 70.843 102.76) (width 0.1) (layer "F.Cu") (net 7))
 (segment (start 58.1375 89.415) (end 62.1776 85.3749) (width 0.1) (layer "B.Cu") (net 7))
 (segment (start 62.1776 85.3749) (end 62.1776 64.8388) (width 0.1) (layer "B.Cu") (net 7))
 (segment (start 62.1776 64.8388) (end 62.1776 64.7754) (width 0.1) (layer "B.Cu") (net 7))
 (segment (start 62.1776 64.7754) (end 69.593 57.36) (width 0.1) (layer "B.Cu") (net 7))
 (segment (start 65.7625 72.6) (end 65.7625 75.1345) (width 0.4) (layer "F.Cu") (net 2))
 (segment (start 65.7625 75.1345) (end 69.578 78.95) (width 0.4) (layer "F.Cu") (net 2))
 (segment (start 69.5775 78.95) (end 72.118 78.95) (width 0.1) (layer "F.Cu") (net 2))
 (segment (start 72.118 78.95) (end 77.198 84.03) (width 0.1) (layer "F.Cu") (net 2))
 (segment (start 60.7225 63.71) (end 60.7225 69.5634) (width 0.4) (layer "B.Cu") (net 2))
 (segment (start 60.7225 69.5634) (end 59.0279 71.2579) (width 0.4) (layer "B.Cu") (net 2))
 (segment (start 59.0279 71.2579) (end 59.0279 71.3329) (width 0.4) (layer "B.Cu") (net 2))
 (segment (start 59.0279 71.3329) (end 59.053 71.358) (width 0.4) (layer "B.Cu") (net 2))
 (segment (start 59.053 71.358) (end 64.521 71.358) (width 0.4) (layer "F.Cu") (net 2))
 (segment (start 64.521 71.358) (end 65.763 72.6) (width 0.4) (layer "F.Cu") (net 2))
 (segment (start 60.7225 63.71) (end 66.012 58.4205) (width 0.4) (layer "F.Cu") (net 2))
 (segment (start 66.012 58.4205) (end 76.1525 58.4205) (width 0.4) (layer "F.Cu") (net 2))
 (segment (start 76.1525 58.4205) (end 77.213 57.36) (width 0.4) (layer "F.Cu") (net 2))
 (segment (start 75.9225 102.76) (end 78.1857 100.4968) (width 0.1) (layer "F.Cu") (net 2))
 (segment (start 78.1857 100.4968) (end 78.1857 85.1977) (width 0.1) (layer "F.Cu") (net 2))
 (segment (start 78.1857 85.1977) (end 78.1857 85.0177) (width 0.1) (layer "F.Cu") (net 2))
 (segment (start 78.1857 85.0177) (end 77.198 84.03) (width 0.1) (layer "F.Cu") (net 2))
 (segment (start 55.6425 106.89) (end 56.6458 105.8867) (width 0.4) (layer "F.Cu") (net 2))
 (segment (start 56.6458 105.8867) (end 75.2268 105.8867) (width 0.4) (layer "F.Cu") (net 2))
 (segment (start 75.2268 105.8867) (end 75.3057 105.8867) (width 0.4) (layer "F.Cu") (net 2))
 (segment (start 75.3057 105.8867) (end 75.6512 106.2322) (width 0.4) (layer "F.Cu") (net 2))
 (segment (start 75.6512 106.2322) (end 75.733 106.175) (width 0.4) (layer "F.Cu") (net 2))
 (segment (start 75.733 106.175) (end 75.733 102.95) (width 0.4) (layer "B.Cu") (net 2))
 (segment (start 75.733 102.95) (end 75.923 102.76) (width 0.4) (layer "B.Cu") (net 2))
 (segment (start 69.5325 106.89) (end 69.5325 106.6105) (width 0.4) (layer "B.Cu") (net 3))
 (segment (start 69.5325 106.6105) (end 73.383 102.76) (width 0.4) (layer "B.Cu") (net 3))
 (segment (start 73.3825 102.76) (end 77.5125 106.89) (width 0.1) (layer "F.Cu") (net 3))
 (segment (start 77.5125 106.89) (end 78.423 106.89) (width 0.1) (layer "F.Cu") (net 3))
 (segment (start 72.0925 57.36) (end 73.0904 56.3621) (width 0.4) (layer "F.Cu") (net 3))
 (segment (start 73.0904 56.3621) (end 78.6789 56.3621) (width 0.4) (layer "F.Cu") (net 3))
 (segment (start 78.6789 56.3621) (end 78.7151 56.3621) (width 0.4) (layer "F.Cu") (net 3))
 (segment (start 78.7151 56.3621) (end 79.713 57.36) (width 0.4) (layer "F.Cu") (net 3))
 (segment (start 69.5775 81.49) (end 74.658 81.49) (width 0.1) (layer "B.Cu") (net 3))
 (segment (start 74.658 81.49) (end 77.198 78.95) (width 0.1) (layer "B.Cu") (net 3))
 (segment (start 60.6425 106.89) (end 61.703 107.9505) (width 0.4) (layer "F.Cu") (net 3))
 (segment (start 61.703 107.9505) (end 68.4725 107.9505) (width 0.4) (layer "F.Cu") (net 3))
 (segment (start 68.4725 107.9505) (end 69.533 106.89) (width 0.4) (layer "F.Cu") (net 3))
 (segment (start 65.7225 63.71) (end 65.743 63.71) (width 0.4) (layer "B.Cu") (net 3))
 (segment (start 65.743 63.71) (end 72.093 57.36) (width 0.4) (layer "B.Cu") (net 3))
 (segment (start 63.2175 89.415) (end 63.2175 83.9768) (width 0.1) (layer "B.Cu") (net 3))
 (segment (start 63.2175 83.9768) (end 66.4431 80.7512) (width 0.1) (layer "B.Cu") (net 3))
 (segment (start 66.4431 80.7512) (end 68.8392 80.7512) (width 0.1) (layer "B.Cu") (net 3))
 (segment (start 68.8392 80.7512) (end 69.578 81.49) (width 0.1) (layer "B.Cu") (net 3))
 (segment (start 63.2175 89.415) (end 63.2175 95.6424) (width 0.1) (layer "B.Cu") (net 3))
 (segment (start 63.2175 95.6424) (end 63.7636 96.1885) (width 0.1) (layer "B.Cu") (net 3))
 (segment (start 63.7636 96.1885) (end 63.7636 96.1976) (width 0.1) (layer "B.Cu") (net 3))
 (segment (start 63.7636 96.1976) (end 63.784 96.218) (width 0.1) (layer "B.Cu") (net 3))
 (segment (start 63.784 96.218) (end 66.841 96.218) (width 0.1) (layer "F.Cu") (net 3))
 (segment (start 66.841 96.218) (end 73.383 102.76) (width 0.1) (layer "F.Cu") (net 3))
 (segment (start 65.7225 63.71) (end 68.4321 66.4196) (width 0.4) (layer "B.Cu") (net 3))
 (segment (start 68.4321 66.4196) (end 68.4321 80.3441) (width 0.4) (layer "B.Cu") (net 3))
 (segment (start 68.4321 80.3441) (end 69.578 81.49) (width 0.4) (layer "B.Cu") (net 3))
 (segment (start 141.9575 80.22) (end 78.468 80.22) (width 0.4) (layer "F.Cu") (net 3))
 (segment (start 78.468 80.22) (end 77.198 78.95) (width 0.4) (layer "F.Cu") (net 3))
 (via (at 66.4415 81.751) (size 0.8) (drill 0.4) (layers "F.Cu" "B.Cu") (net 5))
 (via (at 74.273 97.578) (size 0.8) (drill 0.4) (layers "F.Cu" "B.Cu") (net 5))
 (via (at 75.862 100.0503) (size 0.8) (drill 0.4) (layers "F.Cu" "B.Cu") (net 5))
 (via (at 67.314 86.119) (size 0.8) (drill 0.4) (layers "F.Cu" "B.Cu") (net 4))
 (via (at 66.816 94.443) (size 0.8) (drill 0.4) (layers "F.Cu" "B.Cu") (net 7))
 (via (at 66.816 98.775) (size 0.8) (drill 0.4) (layers "F.Cu" "B.Cu") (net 7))
 (via (at 59.053 71.358) (size 0.8) (drill 0.4) (layers "F.Cu" "B.Cu") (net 2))
 (via (at 75.733 106.175) (size 0.8) (drill 0.4) (layers "F.Cu" "B.Cu") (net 2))
 (via (at 63.784 96.218) (size 0.8) (drill 0.4) (layers "F.Cu" "B.Cu") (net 3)))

